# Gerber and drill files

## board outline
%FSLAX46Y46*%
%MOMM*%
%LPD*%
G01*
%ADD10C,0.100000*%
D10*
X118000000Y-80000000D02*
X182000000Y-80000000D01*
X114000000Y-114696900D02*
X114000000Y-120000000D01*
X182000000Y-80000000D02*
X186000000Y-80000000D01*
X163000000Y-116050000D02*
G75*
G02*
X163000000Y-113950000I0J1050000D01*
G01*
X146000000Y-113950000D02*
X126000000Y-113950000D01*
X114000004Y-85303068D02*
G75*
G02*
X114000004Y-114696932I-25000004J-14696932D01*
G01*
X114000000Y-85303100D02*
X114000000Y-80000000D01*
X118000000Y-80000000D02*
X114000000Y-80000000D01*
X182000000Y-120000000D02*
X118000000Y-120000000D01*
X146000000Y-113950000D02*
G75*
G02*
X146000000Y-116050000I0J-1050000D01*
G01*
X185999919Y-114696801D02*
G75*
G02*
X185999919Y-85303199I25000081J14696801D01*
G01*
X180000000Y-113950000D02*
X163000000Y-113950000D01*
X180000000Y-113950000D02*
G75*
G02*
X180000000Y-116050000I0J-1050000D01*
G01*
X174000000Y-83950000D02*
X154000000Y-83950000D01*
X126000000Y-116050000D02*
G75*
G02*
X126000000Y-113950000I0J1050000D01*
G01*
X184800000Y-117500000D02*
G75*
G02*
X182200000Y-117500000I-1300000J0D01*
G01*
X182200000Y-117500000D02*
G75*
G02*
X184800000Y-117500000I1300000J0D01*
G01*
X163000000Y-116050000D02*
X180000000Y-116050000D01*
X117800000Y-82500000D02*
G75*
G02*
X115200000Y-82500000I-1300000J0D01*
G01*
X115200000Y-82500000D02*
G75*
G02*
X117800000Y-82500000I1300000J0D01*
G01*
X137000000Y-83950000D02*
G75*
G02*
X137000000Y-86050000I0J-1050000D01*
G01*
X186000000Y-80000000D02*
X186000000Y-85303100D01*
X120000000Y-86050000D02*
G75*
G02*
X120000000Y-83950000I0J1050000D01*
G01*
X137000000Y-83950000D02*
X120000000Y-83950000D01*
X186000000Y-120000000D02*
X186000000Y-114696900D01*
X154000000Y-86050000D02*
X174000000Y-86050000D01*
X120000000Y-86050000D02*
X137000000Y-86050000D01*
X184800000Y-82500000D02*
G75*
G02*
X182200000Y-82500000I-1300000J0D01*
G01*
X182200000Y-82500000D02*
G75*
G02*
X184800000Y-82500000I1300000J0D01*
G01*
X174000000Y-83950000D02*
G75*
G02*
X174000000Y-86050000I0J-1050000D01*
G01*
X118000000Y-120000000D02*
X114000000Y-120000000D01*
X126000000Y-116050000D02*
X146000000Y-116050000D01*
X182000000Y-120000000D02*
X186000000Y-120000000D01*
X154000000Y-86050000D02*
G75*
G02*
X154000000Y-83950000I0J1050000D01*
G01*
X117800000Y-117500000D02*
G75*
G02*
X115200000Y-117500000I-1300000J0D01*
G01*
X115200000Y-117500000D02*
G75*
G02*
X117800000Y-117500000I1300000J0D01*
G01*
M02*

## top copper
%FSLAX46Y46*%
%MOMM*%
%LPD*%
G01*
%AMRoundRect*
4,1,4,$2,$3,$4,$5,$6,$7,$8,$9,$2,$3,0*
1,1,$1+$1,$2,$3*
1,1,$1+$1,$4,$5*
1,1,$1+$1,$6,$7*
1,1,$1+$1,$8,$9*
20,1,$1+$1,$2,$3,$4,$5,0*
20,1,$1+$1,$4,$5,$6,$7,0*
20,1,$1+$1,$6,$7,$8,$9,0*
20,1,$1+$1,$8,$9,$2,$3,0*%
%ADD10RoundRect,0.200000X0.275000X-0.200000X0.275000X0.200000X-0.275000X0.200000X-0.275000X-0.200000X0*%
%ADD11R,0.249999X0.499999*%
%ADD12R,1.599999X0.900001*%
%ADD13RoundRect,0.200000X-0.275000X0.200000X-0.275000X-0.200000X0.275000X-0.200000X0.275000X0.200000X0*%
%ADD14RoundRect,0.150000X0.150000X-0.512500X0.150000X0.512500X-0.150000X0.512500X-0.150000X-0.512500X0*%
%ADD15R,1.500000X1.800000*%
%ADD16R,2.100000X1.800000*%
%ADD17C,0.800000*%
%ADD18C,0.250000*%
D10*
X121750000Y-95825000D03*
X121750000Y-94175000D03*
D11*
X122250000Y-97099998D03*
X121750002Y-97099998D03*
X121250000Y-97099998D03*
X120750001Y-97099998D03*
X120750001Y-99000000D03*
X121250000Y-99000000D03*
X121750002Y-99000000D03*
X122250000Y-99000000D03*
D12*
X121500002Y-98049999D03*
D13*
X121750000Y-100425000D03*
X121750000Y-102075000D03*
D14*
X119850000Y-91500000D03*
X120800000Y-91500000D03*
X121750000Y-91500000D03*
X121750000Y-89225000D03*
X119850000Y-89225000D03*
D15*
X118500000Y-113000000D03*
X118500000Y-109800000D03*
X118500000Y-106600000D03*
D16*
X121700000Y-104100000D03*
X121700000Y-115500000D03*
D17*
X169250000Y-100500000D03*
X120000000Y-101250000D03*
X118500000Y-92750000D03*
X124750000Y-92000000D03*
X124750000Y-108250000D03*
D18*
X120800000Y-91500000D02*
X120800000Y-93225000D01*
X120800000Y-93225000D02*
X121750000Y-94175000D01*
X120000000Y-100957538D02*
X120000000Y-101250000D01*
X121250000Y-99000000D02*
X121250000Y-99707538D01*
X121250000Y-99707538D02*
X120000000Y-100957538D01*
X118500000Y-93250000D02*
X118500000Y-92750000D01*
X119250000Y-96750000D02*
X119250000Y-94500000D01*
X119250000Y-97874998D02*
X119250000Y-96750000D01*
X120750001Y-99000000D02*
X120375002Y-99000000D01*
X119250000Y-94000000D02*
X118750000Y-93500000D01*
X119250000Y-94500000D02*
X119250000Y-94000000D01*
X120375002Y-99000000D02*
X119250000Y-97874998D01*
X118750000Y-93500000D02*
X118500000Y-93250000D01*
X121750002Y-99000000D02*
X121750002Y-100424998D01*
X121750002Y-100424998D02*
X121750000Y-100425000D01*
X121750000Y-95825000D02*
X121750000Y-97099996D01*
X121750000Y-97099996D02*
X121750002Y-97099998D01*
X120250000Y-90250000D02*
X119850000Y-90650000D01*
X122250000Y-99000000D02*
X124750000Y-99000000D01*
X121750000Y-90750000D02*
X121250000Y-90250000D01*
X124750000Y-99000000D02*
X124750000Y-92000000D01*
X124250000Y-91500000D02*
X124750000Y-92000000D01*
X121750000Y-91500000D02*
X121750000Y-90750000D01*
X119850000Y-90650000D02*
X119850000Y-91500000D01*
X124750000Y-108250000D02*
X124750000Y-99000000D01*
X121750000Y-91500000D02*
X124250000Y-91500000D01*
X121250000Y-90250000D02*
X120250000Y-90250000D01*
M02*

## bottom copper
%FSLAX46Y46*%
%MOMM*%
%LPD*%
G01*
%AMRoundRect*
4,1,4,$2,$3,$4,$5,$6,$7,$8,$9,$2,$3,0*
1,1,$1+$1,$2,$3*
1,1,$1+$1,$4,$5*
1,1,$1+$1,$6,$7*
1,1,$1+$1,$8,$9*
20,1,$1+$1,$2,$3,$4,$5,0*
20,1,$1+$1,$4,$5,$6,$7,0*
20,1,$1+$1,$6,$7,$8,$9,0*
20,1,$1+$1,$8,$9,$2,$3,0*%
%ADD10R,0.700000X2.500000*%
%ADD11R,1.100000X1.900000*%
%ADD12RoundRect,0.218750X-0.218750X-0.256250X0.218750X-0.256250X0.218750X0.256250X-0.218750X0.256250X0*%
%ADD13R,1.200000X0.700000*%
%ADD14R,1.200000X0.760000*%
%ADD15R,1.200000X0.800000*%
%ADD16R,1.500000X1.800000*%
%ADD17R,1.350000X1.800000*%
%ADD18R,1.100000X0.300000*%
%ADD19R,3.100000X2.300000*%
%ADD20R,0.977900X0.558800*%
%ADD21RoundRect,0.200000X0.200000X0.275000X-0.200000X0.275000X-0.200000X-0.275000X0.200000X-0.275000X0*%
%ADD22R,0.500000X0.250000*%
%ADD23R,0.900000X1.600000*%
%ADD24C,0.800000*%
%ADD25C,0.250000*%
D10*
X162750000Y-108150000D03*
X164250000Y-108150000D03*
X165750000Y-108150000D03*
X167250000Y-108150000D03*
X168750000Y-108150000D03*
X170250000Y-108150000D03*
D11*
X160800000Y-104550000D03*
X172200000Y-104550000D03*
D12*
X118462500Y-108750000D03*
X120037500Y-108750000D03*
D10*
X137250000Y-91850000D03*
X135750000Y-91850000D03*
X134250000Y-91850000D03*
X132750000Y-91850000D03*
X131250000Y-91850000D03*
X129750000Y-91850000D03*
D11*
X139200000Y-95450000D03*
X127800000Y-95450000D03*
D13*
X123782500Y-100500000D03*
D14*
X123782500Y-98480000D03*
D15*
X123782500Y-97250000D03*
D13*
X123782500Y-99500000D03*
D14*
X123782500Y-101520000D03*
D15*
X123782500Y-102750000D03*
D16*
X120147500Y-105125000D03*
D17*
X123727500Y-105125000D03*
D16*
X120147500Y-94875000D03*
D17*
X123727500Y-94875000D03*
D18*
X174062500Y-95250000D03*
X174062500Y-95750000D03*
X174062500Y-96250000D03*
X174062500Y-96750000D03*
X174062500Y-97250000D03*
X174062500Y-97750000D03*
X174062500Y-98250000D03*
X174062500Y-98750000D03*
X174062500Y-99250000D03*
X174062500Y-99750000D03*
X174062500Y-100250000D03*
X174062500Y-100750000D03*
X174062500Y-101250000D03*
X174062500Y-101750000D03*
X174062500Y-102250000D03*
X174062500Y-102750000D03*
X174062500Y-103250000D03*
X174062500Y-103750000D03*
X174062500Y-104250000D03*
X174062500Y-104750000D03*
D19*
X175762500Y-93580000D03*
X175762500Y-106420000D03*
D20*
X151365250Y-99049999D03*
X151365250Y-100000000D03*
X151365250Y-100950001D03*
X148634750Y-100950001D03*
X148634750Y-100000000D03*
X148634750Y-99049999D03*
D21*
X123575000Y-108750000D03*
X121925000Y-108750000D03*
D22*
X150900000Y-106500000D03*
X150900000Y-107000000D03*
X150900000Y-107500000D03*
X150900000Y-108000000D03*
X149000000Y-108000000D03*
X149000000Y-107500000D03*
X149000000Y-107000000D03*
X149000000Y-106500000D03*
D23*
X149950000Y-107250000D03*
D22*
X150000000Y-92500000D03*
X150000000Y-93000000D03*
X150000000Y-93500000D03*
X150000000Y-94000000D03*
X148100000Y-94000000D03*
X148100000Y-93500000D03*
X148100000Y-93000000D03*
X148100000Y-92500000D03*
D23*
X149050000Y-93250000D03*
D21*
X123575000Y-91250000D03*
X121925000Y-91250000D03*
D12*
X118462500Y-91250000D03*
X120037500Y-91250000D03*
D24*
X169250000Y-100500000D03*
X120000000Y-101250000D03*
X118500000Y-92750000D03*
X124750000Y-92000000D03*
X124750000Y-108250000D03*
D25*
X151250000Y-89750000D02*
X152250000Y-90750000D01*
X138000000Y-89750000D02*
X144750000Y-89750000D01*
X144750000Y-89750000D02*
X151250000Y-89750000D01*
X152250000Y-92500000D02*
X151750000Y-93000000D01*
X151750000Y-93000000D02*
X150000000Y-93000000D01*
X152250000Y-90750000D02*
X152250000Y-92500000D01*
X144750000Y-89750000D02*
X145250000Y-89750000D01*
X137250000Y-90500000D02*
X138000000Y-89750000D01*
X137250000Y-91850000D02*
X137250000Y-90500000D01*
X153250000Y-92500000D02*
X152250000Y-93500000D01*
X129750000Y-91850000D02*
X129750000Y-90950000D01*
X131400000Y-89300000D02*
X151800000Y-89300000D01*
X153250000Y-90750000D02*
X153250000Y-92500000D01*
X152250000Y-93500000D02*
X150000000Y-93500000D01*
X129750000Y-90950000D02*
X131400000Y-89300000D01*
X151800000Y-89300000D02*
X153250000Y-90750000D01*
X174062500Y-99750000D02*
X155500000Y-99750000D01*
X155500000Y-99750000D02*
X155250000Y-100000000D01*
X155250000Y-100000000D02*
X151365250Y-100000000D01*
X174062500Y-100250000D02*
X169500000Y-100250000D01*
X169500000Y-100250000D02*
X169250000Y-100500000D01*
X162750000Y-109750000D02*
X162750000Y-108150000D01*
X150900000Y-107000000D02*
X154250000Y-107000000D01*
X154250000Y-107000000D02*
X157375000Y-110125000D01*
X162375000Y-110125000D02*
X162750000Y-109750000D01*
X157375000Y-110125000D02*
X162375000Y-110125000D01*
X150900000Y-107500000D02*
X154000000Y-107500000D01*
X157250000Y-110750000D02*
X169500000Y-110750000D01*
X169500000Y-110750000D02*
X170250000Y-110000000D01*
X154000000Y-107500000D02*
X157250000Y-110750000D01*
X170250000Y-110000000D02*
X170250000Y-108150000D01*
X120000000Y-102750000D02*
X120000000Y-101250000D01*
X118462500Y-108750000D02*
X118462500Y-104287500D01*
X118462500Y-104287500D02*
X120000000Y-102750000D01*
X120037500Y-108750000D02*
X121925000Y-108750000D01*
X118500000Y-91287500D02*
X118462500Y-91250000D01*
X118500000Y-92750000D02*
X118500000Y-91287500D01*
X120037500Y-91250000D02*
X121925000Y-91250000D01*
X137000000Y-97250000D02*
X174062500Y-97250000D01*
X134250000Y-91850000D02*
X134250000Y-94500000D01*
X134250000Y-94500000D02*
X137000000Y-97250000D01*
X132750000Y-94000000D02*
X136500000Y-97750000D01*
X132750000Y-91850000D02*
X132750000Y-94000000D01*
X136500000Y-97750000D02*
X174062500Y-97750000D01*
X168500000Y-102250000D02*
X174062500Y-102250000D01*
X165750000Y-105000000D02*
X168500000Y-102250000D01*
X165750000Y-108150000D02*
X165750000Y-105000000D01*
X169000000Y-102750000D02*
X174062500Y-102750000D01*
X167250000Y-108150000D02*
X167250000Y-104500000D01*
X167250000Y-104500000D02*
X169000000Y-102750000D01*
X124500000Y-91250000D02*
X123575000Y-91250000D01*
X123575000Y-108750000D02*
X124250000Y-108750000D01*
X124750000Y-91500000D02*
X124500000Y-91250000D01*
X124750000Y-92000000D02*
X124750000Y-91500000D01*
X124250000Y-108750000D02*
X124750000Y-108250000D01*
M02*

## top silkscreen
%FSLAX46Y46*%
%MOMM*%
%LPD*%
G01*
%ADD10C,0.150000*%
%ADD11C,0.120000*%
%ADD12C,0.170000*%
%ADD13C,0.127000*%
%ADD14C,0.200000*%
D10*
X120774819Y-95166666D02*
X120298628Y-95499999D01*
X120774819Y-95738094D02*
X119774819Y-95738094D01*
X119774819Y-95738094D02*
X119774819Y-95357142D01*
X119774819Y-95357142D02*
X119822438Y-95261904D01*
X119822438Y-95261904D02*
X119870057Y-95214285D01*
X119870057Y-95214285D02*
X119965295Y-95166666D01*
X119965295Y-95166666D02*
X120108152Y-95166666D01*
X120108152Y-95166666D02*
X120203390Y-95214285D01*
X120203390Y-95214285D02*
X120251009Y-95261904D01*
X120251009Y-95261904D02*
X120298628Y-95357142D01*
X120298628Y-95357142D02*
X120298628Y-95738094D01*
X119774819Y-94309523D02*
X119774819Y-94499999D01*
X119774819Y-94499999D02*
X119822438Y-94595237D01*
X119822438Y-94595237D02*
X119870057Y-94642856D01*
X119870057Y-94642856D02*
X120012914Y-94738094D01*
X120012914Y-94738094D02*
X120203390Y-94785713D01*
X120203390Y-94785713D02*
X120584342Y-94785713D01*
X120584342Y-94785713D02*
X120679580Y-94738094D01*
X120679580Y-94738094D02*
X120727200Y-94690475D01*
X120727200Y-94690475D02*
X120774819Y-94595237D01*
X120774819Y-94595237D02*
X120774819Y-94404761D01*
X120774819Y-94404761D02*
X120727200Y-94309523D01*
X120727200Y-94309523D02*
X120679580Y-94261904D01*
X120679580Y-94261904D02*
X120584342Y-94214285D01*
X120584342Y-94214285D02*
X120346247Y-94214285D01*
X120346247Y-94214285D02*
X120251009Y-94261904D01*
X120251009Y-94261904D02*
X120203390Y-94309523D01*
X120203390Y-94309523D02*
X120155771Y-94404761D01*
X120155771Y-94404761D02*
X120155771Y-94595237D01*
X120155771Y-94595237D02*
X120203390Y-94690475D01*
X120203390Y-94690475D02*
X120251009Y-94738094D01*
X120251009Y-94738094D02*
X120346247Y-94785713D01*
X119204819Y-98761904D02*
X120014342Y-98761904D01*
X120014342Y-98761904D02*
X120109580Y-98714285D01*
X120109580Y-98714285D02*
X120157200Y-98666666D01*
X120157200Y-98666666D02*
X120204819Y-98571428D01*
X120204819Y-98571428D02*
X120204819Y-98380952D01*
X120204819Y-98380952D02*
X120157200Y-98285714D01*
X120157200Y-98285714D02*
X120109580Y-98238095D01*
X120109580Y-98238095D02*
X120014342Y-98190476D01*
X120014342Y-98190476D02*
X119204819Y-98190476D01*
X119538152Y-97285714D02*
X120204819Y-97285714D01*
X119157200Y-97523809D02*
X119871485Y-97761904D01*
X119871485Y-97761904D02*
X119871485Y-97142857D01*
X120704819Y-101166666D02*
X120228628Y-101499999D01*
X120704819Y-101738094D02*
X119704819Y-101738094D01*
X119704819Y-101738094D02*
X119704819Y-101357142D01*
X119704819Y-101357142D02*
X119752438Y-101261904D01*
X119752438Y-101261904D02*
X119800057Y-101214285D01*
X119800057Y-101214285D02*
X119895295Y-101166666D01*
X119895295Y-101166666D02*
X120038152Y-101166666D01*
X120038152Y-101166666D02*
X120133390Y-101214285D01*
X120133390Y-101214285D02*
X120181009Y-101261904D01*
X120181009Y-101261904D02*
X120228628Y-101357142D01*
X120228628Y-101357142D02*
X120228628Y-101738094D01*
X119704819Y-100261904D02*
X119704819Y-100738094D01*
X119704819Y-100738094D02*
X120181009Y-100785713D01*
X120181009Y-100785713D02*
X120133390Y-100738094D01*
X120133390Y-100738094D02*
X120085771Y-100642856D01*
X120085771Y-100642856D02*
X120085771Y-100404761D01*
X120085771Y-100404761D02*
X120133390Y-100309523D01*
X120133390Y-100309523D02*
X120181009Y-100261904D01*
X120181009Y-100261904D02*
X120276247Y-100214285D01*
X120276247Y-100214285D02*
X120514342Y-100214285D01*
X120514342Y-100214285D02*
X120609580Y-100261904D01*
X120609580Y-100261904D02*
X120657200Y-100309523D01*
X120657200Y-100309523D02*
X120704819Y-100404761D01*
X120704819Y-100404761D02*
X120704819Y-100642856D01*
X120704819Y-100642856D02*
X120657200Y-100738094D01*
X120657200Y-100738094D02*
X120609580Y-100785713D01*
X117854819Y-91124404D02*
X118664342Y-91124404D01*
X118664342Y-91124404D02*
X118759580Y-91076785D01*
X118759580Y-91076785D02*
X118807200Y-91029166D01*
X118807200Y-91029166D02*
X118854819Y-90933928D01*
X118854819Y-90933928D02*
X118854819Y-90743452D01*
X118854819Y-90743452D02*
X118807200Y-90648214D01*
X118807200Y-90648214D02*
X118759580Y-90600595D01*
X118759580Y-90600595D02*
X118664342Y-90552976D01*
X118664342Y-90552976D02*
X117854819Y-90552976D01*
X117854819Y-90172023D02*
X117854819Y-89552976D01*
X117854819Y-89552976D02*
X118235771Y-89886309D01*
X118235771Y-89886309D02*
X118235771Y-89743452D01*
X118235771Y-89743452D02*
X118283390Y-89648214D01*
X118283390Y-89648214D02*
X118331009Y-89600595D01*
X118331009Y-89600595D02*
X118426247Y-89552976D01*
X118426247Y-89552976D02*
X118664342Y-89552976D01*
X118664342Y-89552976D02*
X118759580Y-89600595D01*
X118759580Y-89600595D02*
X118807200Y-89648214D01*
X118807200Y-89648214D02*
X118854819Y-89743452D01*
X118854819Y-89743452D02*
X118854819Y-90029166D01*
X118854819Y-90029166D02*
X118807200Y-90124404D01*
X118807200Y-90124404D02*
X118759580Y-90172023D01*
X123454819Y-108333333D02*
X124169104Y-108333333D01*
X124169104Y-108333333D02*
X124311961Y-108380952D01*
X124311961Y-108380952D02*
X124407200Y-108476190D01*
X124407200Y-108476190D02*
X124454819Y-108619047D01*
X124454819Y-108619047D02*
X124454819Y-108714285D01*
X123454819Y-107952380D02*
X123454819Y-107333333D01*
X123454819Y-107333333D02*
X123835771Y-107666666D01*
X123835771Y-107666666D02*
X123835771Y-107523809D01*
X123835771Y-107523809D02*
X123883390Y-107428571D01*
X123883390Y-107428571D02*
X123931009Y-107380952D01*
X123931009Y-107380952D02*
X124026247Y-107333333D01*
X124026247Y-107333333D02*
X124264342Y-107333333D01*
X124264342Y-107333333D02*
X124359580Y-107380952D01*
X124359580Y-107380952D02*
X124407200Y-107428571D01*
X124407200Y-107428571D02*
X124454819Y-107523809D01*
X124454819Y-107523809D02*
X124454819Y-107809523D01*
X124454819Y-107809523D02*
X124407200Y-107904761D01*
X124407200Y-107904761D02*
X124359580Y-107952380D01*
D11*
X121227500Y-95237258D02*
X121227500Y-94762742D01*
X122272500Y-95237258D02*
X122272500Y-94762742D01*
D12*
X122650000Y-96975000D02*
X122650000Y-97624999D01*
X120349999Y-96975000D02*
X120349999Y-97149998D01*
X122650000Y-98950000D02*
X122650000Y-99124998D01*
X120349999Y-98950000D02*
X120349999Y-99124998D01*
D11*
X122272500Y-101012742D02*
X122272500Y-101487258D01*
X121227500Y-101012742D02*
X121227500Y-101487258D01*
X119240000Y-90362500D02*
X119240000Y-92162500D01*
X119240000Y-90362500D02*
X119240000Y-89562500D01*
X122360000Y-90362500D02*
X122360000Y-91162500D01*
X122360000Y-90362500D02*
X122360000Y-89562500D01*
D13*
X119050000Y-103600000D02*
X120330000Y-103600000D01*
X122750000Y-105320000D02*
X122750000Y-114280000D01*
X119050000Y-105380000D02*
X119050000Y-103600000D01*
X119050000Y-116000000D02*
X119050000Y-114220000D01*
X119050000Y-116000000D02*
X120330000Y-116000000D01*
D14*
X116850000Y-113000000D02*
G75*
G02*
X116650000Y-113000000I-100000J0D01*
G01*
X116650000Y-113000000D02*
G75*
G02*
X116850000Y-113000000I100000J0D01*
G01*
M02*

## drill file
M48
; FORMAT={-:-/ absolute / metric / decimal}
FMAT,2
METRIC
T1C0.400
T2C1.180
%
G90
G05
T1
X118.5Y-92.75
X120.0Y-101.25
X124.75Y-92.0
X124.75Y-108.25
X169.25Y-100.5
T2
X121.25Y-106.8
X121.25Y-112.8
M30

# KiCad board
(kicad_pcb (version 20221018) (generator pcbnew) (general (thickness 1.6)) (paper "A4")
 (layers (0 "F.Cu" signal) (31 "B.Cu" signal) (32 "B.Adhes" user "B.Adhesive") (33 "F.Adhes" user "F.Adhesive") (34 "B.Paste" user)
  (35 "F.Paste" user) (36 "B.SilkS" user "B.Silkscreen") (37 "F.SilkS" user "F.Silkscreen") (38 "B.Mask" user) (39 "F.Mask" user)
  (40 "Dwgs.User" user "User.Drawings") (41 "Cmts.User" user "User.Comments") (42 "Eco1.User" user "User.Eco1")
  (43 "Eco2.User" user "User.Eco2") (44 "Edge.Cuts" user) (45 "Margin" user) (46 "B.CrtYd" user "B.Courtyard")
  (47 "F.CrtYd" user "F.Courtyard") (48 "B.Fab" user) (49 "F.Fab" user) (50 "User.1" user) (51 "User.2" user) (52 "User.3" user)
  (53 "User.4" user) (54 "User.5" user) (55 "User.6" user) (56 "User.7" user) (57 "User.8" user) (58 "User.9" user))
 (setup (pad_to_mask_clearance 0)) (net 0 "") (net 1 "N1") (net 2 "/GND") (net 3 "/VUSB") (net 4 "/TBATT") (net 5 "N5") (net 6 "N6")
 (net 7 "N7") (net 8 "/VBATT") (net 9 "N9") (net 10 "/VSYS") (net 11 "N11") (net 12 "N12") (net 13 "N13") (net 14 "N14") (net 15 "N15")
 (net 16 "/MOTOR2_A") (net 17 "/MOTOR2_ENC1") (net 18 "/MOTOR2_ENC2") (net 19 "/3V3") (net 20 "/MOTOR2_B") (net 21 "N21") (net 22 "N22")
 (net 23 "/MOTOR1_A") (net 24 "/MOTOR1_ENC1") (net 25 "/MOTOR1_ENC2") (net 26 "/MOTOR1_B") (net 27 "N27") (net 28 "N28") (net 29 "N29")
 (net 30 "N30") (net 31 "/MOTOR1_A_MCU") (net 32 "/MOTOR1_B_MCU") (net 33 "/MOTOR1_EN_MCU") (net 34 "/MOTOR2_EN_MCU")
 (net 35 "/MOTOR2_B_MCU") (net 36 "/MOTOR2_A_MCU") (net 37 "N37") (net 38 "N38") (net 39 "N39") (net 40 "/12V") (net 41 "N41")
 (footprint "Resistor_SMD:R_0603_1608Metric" (layer "F.Cu") (at 121.75 95 90)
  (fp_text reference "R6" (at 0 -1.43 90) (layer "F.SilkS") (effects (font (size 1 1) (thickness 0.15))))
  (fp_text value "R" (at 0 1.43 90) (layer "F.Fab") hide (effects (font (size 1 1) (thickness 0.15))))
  (fp_line (start -0.237258 -0.5225) (end 0.237258 -0.5225) (stroke (width 0.12) (type solid)) (layer "F.SilkS"))
  (fp_line (start -0.237258 0.5225) (end 0.237258 0.5225) (stroke (width 0.12) (type solid)) (layer "F.SilkS"))
  (pad "1" smd roundrect (at -0.825 0 90) (size 0.8 0.95) (layers "F.Cu" "F.Paste" "F.Mask") (roundrect_rratio 0.25) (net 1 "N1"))
  (pad "2" smd roundrect (at 0.825 0 90) (size 0.8 0.95) (layers "F.Cu" "F.Paste" "F.Mask") (roundrect_rratio 0.25) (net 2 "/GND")))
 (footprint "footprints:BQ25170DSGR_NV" (layer "F.Cu") (at 121.500002 98.049999 -90)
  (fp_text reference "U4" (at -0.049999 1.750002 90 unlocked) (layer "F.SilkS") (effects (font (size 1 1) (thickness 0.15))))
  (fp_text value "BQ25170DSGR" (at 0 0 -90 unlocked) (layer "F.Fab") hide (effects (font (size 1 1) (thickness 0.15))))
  (fp_line (start -1.074999 -1.149998) (end -0.425 -1.149998) (stroke (width 0.17) (type solid)) (layer "F.SilkS"))
  (fp_line (start -1.074999 1.150003) (end -0.900001 1.150003) (stroke (width 0.17) (type solid)) (layer "F.SilkS"))
  (fp_line (start 0.900001 -1.149998) (end 1.074999 -1.149998) (stroke (width 0.17) (type solid)) (layer "F.SilkS"))
  (fp_line (start 0.900001 1.150003) (end 1.074999 1.150003) (stroke (width 0.17) (type solid)) (layer "F.SilkS"))
  (pad "1" smd rect (at -0.950001 -0.749998) (size 0.249999 0.499999) (layers "F.Cu" "F.Paste" "F.Mask") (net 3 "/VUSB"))
  (pad "2" smd rect (at -0.950001 -0.25) (size 0.249999 0.499999) (layers "F.Cu" "F.Paste" "F.Mask") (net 1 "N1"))
  (pad "3" smd rect (at -0.950001 0.250002) (size 0.249999 0.499999) (layers "F.Cu" "F.Paste" "F.Mask") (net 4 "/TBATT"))
  (pad "4" smd rect (at -0.950001 0.750001) (size 0.249999 0.499999) (layers "F.Cu" "F.Paste" "F.Mask") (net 2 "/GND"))
  (pad "5" smd rect (at 0.950001 0.750001) (size 0.249999 0.499999) (layers "F.Cu" "F.Paste" "F.Mask") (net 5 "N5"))
  (pad "6" smd rect (at 0.950001 0.250002) (size 0.249999 0.499999) (layers "F.Cu" "F.Paste" "F.Mask") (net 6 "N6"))
  (pad "7" smd rect (at 0.950001 -0.25) (size 0.249999 0.499999) (layers "F.Cu" "F.Paste" "F.Mask") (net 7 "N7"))
  (pad "8" smd rect (at 0.950001 -0.749998) (size 0.249999 0.499999) (layers "F.Cu" "F.Paste" "F.Mask") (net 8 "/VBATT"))
  (pad "9" smd rect (at 0 0 270) (size 0.900001 1.599999) (layers "F.Cu" "F.Paste" "F.Mask") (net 2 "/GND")))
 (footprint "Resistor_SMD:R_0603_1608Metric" (layer "F.Cu") (at 121.75 101.25 -90)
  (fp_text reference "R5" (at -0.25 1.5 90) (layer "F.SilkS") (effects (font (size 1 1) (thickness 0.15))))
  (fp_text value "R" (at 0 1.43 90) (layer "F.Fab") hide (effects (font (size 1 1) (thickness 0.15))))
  (fp_line (start -0.237258 -0.5225) (end 0.237258 -0.5225) (stroke (width 0.12) (type solid)) (layer "F.SilkS"))
  (fp_line (start -0.237258 0.5225) (end 0.237258 0.5225) (stroke (width 0.12) (type solid)) (layer "F.SilkS"))
  (pad "1" smd roundrect (at -0.825 0 270) (size 0.8 0.95) (layers "F.Cu" "F.Paste" "F.Mask") (roundrect_rratio 0.25) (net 7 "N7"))
  (pad "2" smd roundrect (at 0.825 0 270) (size 0.8 0.95) (layers "F.Cu" "F.Paste" "F.Mask") (roundrect_rratio 0.25) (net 2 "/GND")))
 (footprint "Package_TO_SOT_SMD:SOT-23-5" (layer "F.Cu") (at 120.8 90.3625 90)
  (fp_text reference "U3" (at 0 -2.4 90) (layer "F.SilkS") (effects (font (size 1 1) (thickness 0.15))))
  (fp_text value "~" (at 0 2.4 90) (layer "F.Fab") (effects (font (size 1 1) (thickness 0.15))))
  (fp_line (start 0 -1.56) (end -1.8 -1.56) (stroke (width 0.12) (type solid)) (layer "F.SilkS"))
  (fp_line (start 0 -1.56) (end 0.8 -1.56) (stroke (width 0.12) (type solid)) (layer "F.SilkS"))
  (fp_line (start 0 1.56) (end -0.8 1.56) (stroke (width 0.12) (type solid)) (layer "F.SilkS"))
  (fp_line (start 0 1.56) (end 0.8 1.56) (stroke (width 0.12) (type solid)) (layer "F.SilkS"))
  (pad "1" smd roundrect (at -1.1375 -0.95 90) (size 1.325 0.6) (layers "F.Cu" "F.Paste" "F.Mask") (roundrect_rratio 0.25) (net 8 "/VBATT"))
  (pad "2" smd roundrect (at -1.1375 0 90) (size 1.325 0.6) (layers "F.Cu" "F.Paste" "F.Mask") (roundrect_rratio 0.25) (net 2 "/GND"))
  (pad "3" smd roundrect (at -1.1375 0.95 90) (size 1.325 0.6) (layers "F.Cu" "F.Paste" "F.Mask") (roundrect_rratio 0.25) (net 8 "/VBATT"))
  (pad "4" smd roundrect (at 1.1375 0.95 90) (size 1.325 0.6) (layers "F.Cu" "F.Paste" "F.Mask") (roundrect_rratio 0.25) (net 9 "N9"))
  (pad "5" smd roundrect (at 1.1375 -0.95 90) (size 1.325 0.6) (layers "F.Cu" "F.Paste" "F.Mask") (roundrect_rratio 0.25) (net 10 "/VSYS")))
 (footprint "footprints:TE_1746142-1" (layer "F.Cu") (at 121.25 109.8 -90)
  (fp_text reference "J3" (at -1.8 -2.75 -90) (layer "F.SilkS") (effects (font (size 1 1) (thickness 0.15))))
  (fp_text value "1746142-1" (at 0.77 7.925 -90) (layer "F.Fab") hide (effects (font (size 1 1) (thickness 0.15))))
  (fp_line (start -6.2 2.2) (end -6.2 0.92) (stroke (width 0.127) (type solid)) (layer "F.SilkS"))
  (fp_line (start -4.48 -1.5) (end 4.48 -1.5) (stroke (width 0.127) (type solid)) (layer "F.SilkS"))
  (fp_line (start -4.42 2.2) (end -6.2 2.2) (stroke (width 0.127) (type solid)) (layer "F.SilkS"))
  (fp_line (start 6.2 2.2) (end 4.42 2.2) (stroke (width 0.127) (type solid)) (layer "F.SilkS"))
  (fp_line (start 6.2 2.2) (end 6.2 0.92) (stroke (width 0.127) (type solid)) (layer "F.SilkS"))
  (fp_circle (center 3.2 4.5) (end 3.3 4.5) (stroke (width 0.2) (type solid)) (fill none) (layer "F.SilkS"))
  (pad "" np_thru_hole circle (at -3 0 270) (size 1.18 1.18) (drill 1.18) (layers "*.Cu" "*.Mask"))
  (pad "" np_thru_hole circle (at 3 0 270) (size 1.18 1.18) (drill 1.18) (layers "*.Cu" "*.Mask"))
  (pad "1" smd rect (at 3.2 2.75 270) (size 1.8 1.5) (layers "F.Cu" "F.Paste" "F.Mask") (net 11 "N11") (solder_mask_margin 0.102))
  (pad "2" smd rect (at 0 2.75 270) (size 1.8 1.5) (layers "F.Cu" "F.Paste" "F.Mask") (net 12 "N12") (solder_mask_margin 0.102))
  (pad "3" smd rect (at -3.2 2.75 270) (size 1.8 1.5) (layers "F.Cu" "F.Paste" "F.Mask") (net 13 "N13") (solder_mask_margin 0.102))
  (pad "SH1" smd rect (at -5.7 -0.45 270) (size 1.8 2.1) (layers "F.Cu" "F.Paste" "F.Mask") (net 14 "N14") (solder_mask_margin 0.102))
  (pad "SH2" smd rect (at 5.7 -0.45 270) (size 1.8 2.1) (layers "F.Cu" "F.Paste" "F.Mask") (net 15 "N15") (solder_mask_margin 0.102)))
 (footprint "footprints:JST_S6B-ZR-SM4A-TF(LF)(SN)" (layer "B.Cu") (at 166.5 108.15)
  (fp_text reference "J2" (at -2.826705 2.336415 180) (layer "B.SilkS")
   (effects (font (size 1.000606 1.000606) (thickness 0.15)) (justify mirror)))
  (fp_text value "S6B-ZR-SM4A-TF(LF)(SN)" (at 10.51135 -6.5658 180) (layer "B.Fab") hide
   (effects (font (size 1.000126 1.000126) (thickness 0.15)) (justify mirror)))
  (pad "1" smd rect (at -3.75 0) (size 0.7 2.5) (layers "B.Cu" "B.Paste" "B.Mask") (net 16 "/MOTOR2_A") (solder_mask_margin 0.102))
  (pad "2" smd rect (at -2.25 0) (size 0.7 2.5) (layers "B.Cu" "B.Paste" "B.Mask") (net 2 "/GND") (solder_mask_margin 0.102))
  (pad "3" smd rect (at -0.75 0) (size 0.7 2.5) (layers "B.Cu" "B.Paste" "B.Mask") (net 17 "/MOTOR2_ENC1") (solder_mask_margin 0.102))
  (pad "4" smd rect (at 0.75 0) (size 0.7 2.5) (layers "B.Cu" "B.Paste" "B.Mask") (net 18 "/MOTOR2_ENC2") (solder_mask_margin 0.102))
  (pad "5" smd rect (at 2.25 0) (size 0.7 2.5) (layers "B.Cu" "B.Paste" "B.Mask") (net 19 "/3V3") (solder_mask_margin 0.102))
  (pad "6" smd rect (at 3.75 0) (size 0.7 2.5) (layers "B.Cu" "B.Paste" "B.Mask") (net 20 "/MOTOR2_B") (solder_mask_margin 0.102))
  (pad "SH1" smd rect (at -5.7 -3.6) (size 1.1 1.9) (layers "B.Cu" "B.Paste" "B.Mask") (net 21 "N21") (solder_mask_margin 0.102))
  (pad "SH2" smd rect (at 5.7 -3.6) (size 1.1 1.9) (layers "B.Cu" "B.Paste" "B.Mask") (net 21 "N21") (solder_mask_margin 0.102)))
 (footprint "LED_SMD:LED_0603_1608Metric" (layer "B.Cu") (at 119.25 108.75)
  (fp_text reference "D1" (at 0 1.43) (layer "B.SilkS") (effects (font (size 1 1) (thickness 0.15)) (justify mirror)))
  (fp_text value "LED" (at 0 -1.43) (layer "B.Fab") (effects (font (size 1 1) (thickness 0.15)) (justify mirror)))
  (pad "1" smd roundrect (at -0.7875 0) (size 0.875 0.95) (layers "B.Cu" "B.Paste" "B.Mask") (roundrect_rratio 0.25) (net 6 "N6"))
  (pad "2" smd roundrect (at 0.7875 0) (size 0.875 0.95) (layers "B.Cu" "B.Paste" "B.Mask") (roundrect_rratio 0.25) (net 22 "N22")))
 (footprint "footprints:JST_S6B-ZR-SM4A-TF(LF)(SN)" (layer "B.Cu") (at 133.5 91.85 180)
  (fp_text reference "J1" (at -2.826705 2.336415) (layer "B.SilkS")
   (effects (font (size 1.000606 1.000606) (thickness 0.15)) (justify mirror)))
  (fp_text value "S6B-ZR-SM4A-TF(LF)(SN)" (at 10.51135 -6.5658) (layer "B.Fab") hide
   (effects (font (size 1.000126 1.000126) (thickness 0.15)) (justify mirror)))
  (pad "1" smd rect (at -3.75 0 180) (size 0.7 2.5) (layers "B.Cu" "B.Paste" "B.Mask") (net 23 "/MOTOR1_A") (solder_mask_margin 0.102))
  (pad "2" smd rect (at -2.25 0 180) (size 0.7 2.5) (layers "B.Cu" "B.Paste" "B.Mask") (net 2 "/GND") (solder_mask_margin 0.102))
  (pad "3" smd rect (at -0.75 0 180) (size 0.7 2.5) (layers "B.Cu" "B.Paste" "B.Mask") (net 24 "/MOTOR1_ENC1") (solder_mask_margin 0.102))
  (pad "4" smd rect (at 0.75 0 180) (size 0.7 2.5) (layers "B.Cu" "B.Paste" "B.Mask") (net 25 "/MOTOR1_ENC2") (solder_mask_margin 0.102))
  (pad "5" smd rect (at 2.25 0 180) (size 0.7 2.5) (layers "B.Cu" "B.Paste" "B.Mask") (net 19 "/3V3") (solder_mask_margin 0.102))
  (pad "6" smd rect (at 3.75 0 180) (size 0.7 2.5) (layers "B.Cu" "B.Paste" "B.Mask") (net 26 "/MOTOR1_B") (solder_mask_margin 0.102))
  (pad "SH1" smd rect (at -5.7 -3.6 180) (size 1.1 1.9) (layers "B.Cu" "B.Paste" "B.Mask") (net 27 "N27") (solder_mask_margin 0.102))
  (pad "SH2" smd rect (at 5.7 -3.6 180) (size 1.1 1.9) (layers "B.Cu" "B.Paste" "B.Mask") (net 27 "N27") (solder_mask_margin 0.102)))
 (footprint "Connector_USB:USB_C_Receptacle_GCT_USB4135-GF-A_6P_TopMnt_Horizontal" (layer "B.Cu") (at 120.75 100 90)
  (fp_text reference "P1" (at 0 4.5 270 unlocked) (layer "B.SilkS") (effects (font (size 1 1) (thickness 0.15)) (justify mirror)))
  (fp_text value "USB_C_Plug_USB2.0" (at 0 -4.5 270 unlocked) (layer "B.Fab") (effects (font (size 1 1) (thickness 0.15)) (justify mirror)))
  (pad "A5" smd rect (at -0.5 3.0325 90) (size 0.7 1.2) (layers "B.Cu" "B.Paste" "B.Mask") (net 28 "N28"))
  (pad "A9" smd rect (at 1.52 3.0325 270) (size 0.76 1.2) (layers "B.Cu" "B.Paste" "B.Mask") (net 3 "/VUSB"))
  (pad "A12" smd rect (at 2.75 3.0325 270) (size 0.8 1.2) (layers "B.Cu" "B.Paste" "B.Mask") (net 2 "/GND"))
  (pad "B5" smd rect (at 0.5 3.0325 270) (size 0.7 1.2) (layers "B.Cu" "B.Paste" "B.Mask") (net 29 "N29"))
  (pad "B9" smd rect (at -1.52 3.0325 90) (size 0.76 1.2) (layers "B.Cu" "B.Paste" "B.Mask") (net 3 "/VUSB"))
  (pad "B12" smd rect (at -2.75 3.0325 90) (size 0.8 1.2) (layers "B.Cu" "B.Paste" "B.Mask") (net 2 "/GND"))
  (pad "S1" smd rect (at -5.125 -0.6025 90) (size 1.8 1.5) (layers "B.Cu" "B.Paste" "B.Mask") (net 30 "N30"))
  (pad "S1" smd rect (at -5.125 2.9775 90) (size 1.8 1.35) (layers "B.Cu" "B.Paste" "B.Mask") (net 30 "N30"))
  (pad "S1" smd rect (at 5.125 -0.6025 90) (size 1.8 1.5) (layers "B.Cu" "B.Paste" "B.Mask") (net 30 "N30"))
  (pad "S1" smd rect (at 5.125 2.9775 90) (size 1.8 1.35) (layers "B.Cu" "B.Paste" "B.Mask") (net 30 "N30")))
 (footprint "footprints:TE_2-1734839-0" (layer "B.Cu") (at 174.0625 100 -90)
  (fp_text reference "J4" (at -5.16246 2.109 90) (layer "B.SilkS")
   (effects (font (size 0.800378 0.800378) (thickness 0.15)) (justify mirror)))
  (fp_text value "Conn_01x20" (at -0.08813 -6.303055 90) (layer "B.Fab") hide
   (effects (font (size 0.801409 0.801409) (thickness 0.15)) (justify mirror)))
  (pad "1" smd rect (at -4.75 0 270) (size 0.3 1.1) (layers "B.Cu" "B.Paste" "B.Mask") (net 10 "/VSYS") (solder_mask_margin 0.102))
  (pad "2" smd rect (at -4.25 0 270) (size 0.3 1.1) (layers "B.Cu" "B.Paste" "B.Mask") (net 10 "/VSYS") (solder_mask_margin 0.102))
  (pad "3" smd rect (at -3.75 0 270) (size 0.3 1.1) (layers "B.Cu" "B.Paste" "B.Mask") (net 2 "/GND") (solder_mask_margin 0.102))
  (pad "4" smd rect (at -3.25 0 270) (size 0.3 1.1) (layers "B.Cu" "B.Paste" "B.Mask") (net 2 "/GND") (solder_mask_margin 0.102))
  (pad "5" smd rect (at -2.75 0 270) (size 0.3 1.1) (layers "B.Cu" "B.Paste" "B.Mask") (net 24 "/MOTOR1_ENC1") (solder_mask_margin 0.102))
  (pad "6" smd rect (at -2.25 0 270) (size 0.3 1.1) (layers "B.Cu" "B.Paste" "B.Mask") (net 25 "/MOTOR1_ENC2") (solder_mask_margin 0.102))
  (pad "7" smd rect (at -1.75 0 270) (size 0.3 1.1) (layers "B.Cu" "B.Paste" "B.Mask") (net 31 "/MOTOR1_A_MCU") (solder_mask_margin 0.102))
  (pad "8" smd rect (at -1.25 0 270) (size 0.3 1.1) (layers "B.Cu" "B.Paste" "B.Mask") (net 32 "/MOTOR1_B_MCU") (solder_mask_margin 0.102))
  (pad "9" smd rect (at -0.75 0 270) (size 0.3 1.1) (layers "B.Cu" "B.Paste" "B.Mask") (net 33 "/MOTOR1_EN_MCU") (solder_mask_margin 0.102))
  (pad "10" smd rect (at -0.25 0 270) (size 0.3 1.1) (layers "B.Cu" "B.Paste" "B.Mask") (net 2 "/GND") (solder_mask_margin 0.102))
  (pad "11" smd rect (at 0.25 0 270) (size 0.3 1.1) (layers "B.Cu" "B.Paste" "B.Mask") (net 19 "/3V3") (solder_mask_margin 0.102))
  (pad "12" smd rect (at 0.75 0 270) (size 0.3 1.1) (layers "B.Cu" "B.Paste" "B.Mask") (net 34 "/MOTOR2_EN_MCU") (solder_mask_margin 0.102))
  (pad "13" smd rect (at 1.25 0 270) (size 0.3 1.1) (layers "B.Cu" "B.Paste" "B.Mask") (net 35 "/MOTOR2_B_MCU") (solder_mask_margin 0.102))
  (pad "14" smd rect (at 1.75 0 270) (size 0.3 1.1) (layers "B.Cu" "B.Paste" "B.Mask") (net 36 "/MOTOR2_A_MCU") (solder_mask_margin 0.102))
  (pad "15" smd rect (at 2.25 0 270) (size 0.3 1.1) (layers "B.Cu" "B.Paste" "B.Mask") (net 17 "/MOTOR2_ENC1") (solder_mask_margin 0.102))
  (pad "16" smd rect (at 2.75 0 270) (size 0.3 1.1) (layers "B.Cu" "B.Paste" "B.Mask") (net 18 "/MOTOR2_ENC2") (solder_mask_margin 0.102))
  (pad "17" smd rect (at 3.25 0 270) (size 0.3 1.1) (layers "B.Cu" "B.Paste" "B.Mask") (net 2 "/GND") (solder_mask_margin 0.102))
  (pad "18" smd rect (at 3.75 0 270) (size 0.3 1.1) (layers "B.Cu" "B.Paste" "B.Mask") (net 2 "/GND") (solder_mask_margin 0.102))
  (pad "19" smd rect (at 4.25 0 270) (size 0.3 1.1) (layers "B.Cu" "B.Paste" "B.Mask") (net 3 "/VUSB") (solder_mask_margin 0.102))
  (pad "20" smd rect (at 4.75 0 270) (size 0.3 1.1) (layers "B.Cu" "B.Paste" "B.Mask") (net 3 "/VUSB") (solder_mask_margin 0.102))
  (pad "S1" smd rect (at -6.42 -1.7 270) (size 2.3 3.1) (layers "B.Cu" "B.Paste" "B.Mask") (solder_mask_margin 0.102))
  (pad "S2" smd rect (at 6.42 -1.7 270) (size 2.3 3.1) (layers "B.Cu" "B.Paste" "B.Mask") (solder_mask_margin 0.102)))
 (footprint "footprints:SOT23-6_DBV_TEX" (layer "B.Cu") (at 150 100 180)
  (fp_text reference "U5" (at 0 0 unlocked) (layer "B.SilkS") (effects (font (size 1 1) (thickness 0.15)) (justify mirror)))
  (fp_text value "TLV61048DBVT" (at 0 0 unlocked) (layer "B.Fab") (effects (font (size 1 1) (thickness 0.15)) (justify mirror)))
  (pad "1" smd rect (at -1.36525 0.950001 180) (size 0.9779 0.5588) (layers "B.Cu" "B.Paste" "B.Mask") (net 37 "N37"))
  (pad "2" smd rect (at -1.36525 0 180) (size 0.9779 0.5588) (layers "B.Cu" "B.Paste" "B.Mask") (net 2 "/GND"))
  (pad "3" smd rect (at -1.36525 -0.950001 180) (size 0.9779 0.5588) (layers "B.Cu" "B.Paste" "B.Mask") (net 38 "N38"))
  (pad "4" smd rect (at 1.36525 -0.950001 180) (size 0.9779 0.5588) (layers "B.Cu" "B.Paste" "B.Mask") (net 10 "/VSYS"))
  (pad "5" smd rect (at 1.36525 0 180) (size 0.9779 0.5588) (layers "B.Cu" "B.Paste" "B.Mask") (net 10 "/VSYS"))
  (pad "6" smd rect (at 1.36525 0.950001 180) (size 0.9779 0.5588) (layers "B.Cu" "B.Paste" "B.Mask") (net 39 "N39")))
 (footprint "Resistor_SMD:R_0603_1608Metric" (layer "B.Cu") (at 122.75 108.75 180)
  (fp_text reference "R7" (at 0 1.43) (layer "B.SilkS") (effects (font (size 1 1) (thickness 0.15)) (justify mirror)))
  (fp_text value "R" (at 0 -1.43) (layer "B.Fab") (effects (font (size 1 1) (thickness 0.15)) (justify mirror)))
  (pad "1" smd roundrect (at -0.825 0 180) (size 0.8 0.95) (layers "B.Cu" "B.Paste" "B.Mask") (roundrect_rratio 0.25) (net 8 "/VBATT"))
  (pad "2" smd roundrect (at 0.825 0 180) (size 0.8 0.95) (layers "B.Cu" "B.Paste" "B.Mask") (roundrect_rratio 0.25) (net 22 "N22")))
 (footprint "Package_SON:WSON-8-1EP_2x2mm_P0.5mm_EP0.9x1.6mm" (layer "B.Cu") (at 149.95 107.25 180)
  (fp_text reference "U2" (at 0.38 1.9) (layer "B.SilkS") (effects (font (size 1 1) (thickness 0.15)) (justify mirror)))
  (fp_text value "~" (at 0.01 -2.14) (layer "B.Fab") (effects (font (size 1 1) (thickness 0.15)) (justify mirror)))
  (pad "" smd rect (at 0 -0.4 180) (size 0.75 0.65) (layers "B.Paste"))
  (pad "" smd rect (at 0 0.4 180) (size 0.75 0.65) (layers "B.Paste"))
  (pad "1" smd rect (at -0.95 0.75 180) (size 0.5 0.25) (layers "B.Cu" "B.Paste" "B.Mask") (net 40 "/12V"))
  (pad "2" smd rect (at -0.95 0.25 180) (size 0.5 0.25) (layers "B.Cu" "B.Paste" "B.Mask") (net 16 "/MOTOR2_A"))
  (pad "3" smd rect (at -0.95 -0.25 180) (size 0.5 0.25) (layers "B.Cu" "B.Paste" "B.Mask") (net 20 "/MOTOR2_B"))
  (pad "4" smd rect (at -0.95 -0.75 180) (size 0.5 0.25) (layers "B.Cu" "B.Paste" "B.Mask") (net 2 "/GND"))
  (pad "5" smd rect (at 0.95 -0.75 180) (size 0.5 0.25) (layers "B.Cu" "B.Paste" "B.Mask") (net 35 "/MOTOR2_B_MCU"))
  (pad "6" smd rect (at 0.95 -0.25 180) (size 0.5 0.25) (layers "B.Cu" "B.Paste" "B.Mask") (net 36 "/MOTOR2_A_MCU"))
  (pad "7" smd rect (at 0.95 0.25 180) (size 0.5 0.25) (layers "B.Cu" "B.Paste" "B.Mask") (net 34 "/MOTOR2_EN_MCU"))
  (pad "8" smd rect (at 0.95 0.75 180) (size 0.5 0.25) (layers "B.Cu" "B.Paste" "B.Mask") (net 19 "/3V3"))
  (pad "9" smd rect (at 0 0 180) (size 0.9 1.6) (layers "B.Cu" "B.Mask") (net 2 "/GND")))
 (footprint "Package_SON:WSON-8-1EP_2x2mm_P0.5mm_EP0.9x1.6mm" (layer "B.Cu") (at 149.05 93.25 180)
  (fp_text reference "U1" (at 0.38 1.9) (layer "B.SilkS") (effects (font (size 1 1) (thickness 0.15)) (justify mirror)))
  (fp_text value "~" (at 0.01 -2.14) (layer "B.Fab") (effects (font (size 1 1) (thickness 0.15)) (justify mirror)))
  (pad "" smd rect (at 0 -0.4 180) (size 0.75 0.65) (layers "B.Paste"))
  (pad "" smd rect (at 0 0.4 180) (size 0.75 0.65) (layers "B.Paste"))
  (pad "1" smd rect (at -0.95 0.75 180) (size 0.5 0.25) (layers "B.Cu" "B.Paste" "B.Mask") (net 40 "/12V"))
  (pad "2" smd rect (at -0.95 0.25 180) (size 0.5 0.25) (layers "B.Cu" "B.Paste" "B.Mask") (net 23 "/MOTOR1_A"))
  (pad "3" smd rect (at -0.95 -0.25 180) (size 0.5 0.25) (layers "B.Cu" "B.Paste" "B.Mask") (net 26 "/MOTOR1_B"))
  (pad "4" smd rect (at -0.95 -0.75 180) (size 0.5 0.25) (layers "B.Cu" "B.Paste" "B.Mask") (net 2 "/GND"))
  (pad "5" smd rect (at 0.95 -0.75 180) (size 0.5 0.25) (layers "B.Cu" "B.Paste" "B.Mask") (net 32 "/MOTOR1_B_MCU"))
  (pad "6" smd rect (at 0.95 -0.25 180) (size 0.5 0.25) (layers "B.Cu" "B.Paste" "B.Mask") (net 31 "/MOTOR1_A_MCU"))
  (pad "7" smd rect (at 0.95 0.25 180) (size 0.5 0.25) (layers "B.Cu" "B.Paste" "B.Mask") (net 33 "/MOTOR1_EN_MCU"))
  (pad "8" smd rect (at 0.95 0.75 180) (size 0.5 0.25) (layers "B.Cu" "B.Paste" "B.Mask") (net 19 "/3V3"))
  (pad "9" smd rect (at 0 0 180) (size 0.9 1.6) (layers "B.Cu" "B.Mask") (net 2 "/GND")))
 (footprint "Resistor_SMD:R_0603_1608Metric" (layer "B.Cu") (at 122.75 91.25 180)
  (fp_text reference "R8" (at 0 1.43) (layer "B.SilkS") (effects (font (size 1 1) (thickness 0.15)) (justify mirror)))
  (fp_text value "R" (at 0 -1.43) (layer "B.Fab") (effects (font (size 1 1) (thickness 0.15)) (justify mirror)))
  (pad "1" smd roundrect (at -0.825 0 180) (size 0.8 0.95) (layers "B.Cu" "B.Paste" "B.Mask") (roundrect_rratio 0.25) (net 8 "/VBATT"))
  (pad "2" smd roundrect (at 0.825 0 180) (size 0.8 0.95) (layers "B.Cu" "B.Paste" "B.Mask") (roundrect_rratio 0.25) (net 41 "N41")))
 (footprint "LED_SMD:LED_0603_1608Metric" (layer "B.Cu") (at 119.25 91.25)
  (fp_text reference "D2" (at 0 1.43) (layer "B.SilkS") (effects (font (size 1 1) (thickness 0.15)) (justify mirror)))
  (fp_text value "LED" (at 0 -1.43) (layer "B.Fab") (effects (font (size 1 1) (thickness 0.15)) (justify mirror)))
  (pad "1" smd roundrect (at -0.7875 0) (size 0.875 0.95) (layers "B.Cu" "B.Paste" "B.Mask") (roundrect_rratio 0.25) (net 5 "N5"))
  (pad "2" smd roundrect (at 0.7875 0) (size 0.875 0.95) (layers "B.Cu" "B.Paste" "B.Mask") (roundrect_rratio 0.25) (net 41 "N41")))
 (gr_line (start 118 80) (end 182 80) (stroke (width 0.1) (type solid)) (layer "Edge.Cuts"))
 (gr_line (start 114 114.6969) (end 114 120) (stroke (width 0.1) (type solid)) (layer "Edge.Cuts"))
 (gr_line (start 182 80) (end 186 80) (stroke (width 0.1) (type solid)) (layer "Edge.Cuts"))
 (gr_arc (start 163 116.05) (mid 161.95 115) (end 163 113.95) (stroke (width 0.1) (type solid)) (layer "Edge.Cuts"))
 (gr_line (start 146 113.95) (end 126 113.95) (stroke (width 0.1) (type solid)) (layer "Edge.Cuts"))
 (gr_arc (start 114.000004 85.303068) (mid 118 100) (end 114.000004 114.696932) (stroke (width 0.1) (type solid)) (layer "Edge.Cuts"))
 (gr_line (start 114 85.3031) (end 114 80) (stroke (width 0.1) (type solid)) (layer "Edge.Cuts"))
 (gr_line (start 118 80) (end 114 80) (stroke (width 0.1) (type solid)) (layer "Edge.Cuts"))
 (gr_line (start 182 120) (end 118 120) (stroke (width 0.1) (type solid)) (layer "Edge.Cuts"))
 (gr_arc (start 146 113.95) (mid 147.05 115) (end 146 116.05) (stroke (width 0.1) (type solid)) (layer "Edge.Cuts"))
 (gr_arc (start 185.999919 114.696801) (mid 182 100) (end 185.999919 85.303199) (stroke (width 0.1) (type solid)) (layer "Edge.Cuts"))
 (gr_line (start 180 113.95) (end 163 113.95) (stroke (width 0.1) (type solid)) (layer "Edge.Cuts"))
 (gr_arc (start 180 113.95) (mid 181.05 115) (end 180 116.05) (stroke (width 0.1) (type solid)) (layer "Edge.Cuts"))
 (gr_line (start 174 83.95) (end 154 83.95) (stroke (width 0.1) (type solid)) (layer "Edge.Cuts"))
 (gr_arc (start 126 116.05) (mid 124.95 115) (end 126 113.95) (stroke (width 0.1) (type solid)) (layer "Edge.Cuts"))
 (gr_circle (center 183.5 117.5) (end 184.8 117.5) (stroke (width 0.1) (type solid)) (fill none) (layer "Edge.Cuts"))
 (gr_line (start 163 116.05) (end 180 116.05) (stroke (width 0.1) (type solid)) (layer "Edge.Cuts"))
 (gr_circle (center 116.5 82.5) (end 117.8 82.5) (stroke (width 0.1) (type solid)) (fill none) (layer "Edge.Cuts"))
 (gr_arc (start 137 83.95) (mid 138.05 85) (end 137 86.05) (stroke (width 0.1) (type solid)) (layer "Edge.Cuts"))
 (gr_line (start 186 80) (end 186 85.3031) (stroke (width 0.1) (type solid)) (layer "Edge.Cuts"))
 (gr_arc (start 120 86.05) (mid 118.95 85) (end 120 83.95) (stroke (width 0.1) (type solid)) (layer "Edge.Cuts"))
 (gr_line (start 137 83.95) (end 120 83.95) (stroke (width 0.1) (type solid)) (layer "Edge.Cuts"))
 (gr_line (start 186 120) (end 186 114.6969) (stroke (width 0.1) (type solid)) (layer "Edge.Cuts"))
 (gr_line (start 154 86.05) (end 174 86.05) (stroke (width 0.1) (type solid)) (layer "Edge.Cuts"))
 (gr_line (start 120 86.05) (end 137 86.05) (stroke (width 0.1) (type solid)) (layer "Edge.Cuts"))
 (gr_circle (center 183.5 82.5) (end 184.8 82.5) (stroke (width 0.1) (type solid)) (fill none) (layer "Edge.Cuts"))
 (gr_arc (start 174 83.95) (mid 175.05 85) (end 174 86.05) (stroke (width 0.1) (type solid)) (layer "Edge.Cuts"))
 (gr_line (start 118 120) (end 114 120) (stroke (width 0.1) (type solid)) (layer "Edge.Cuts"))
 (gr_line (start 126 116.05) (end 146 116.05) (stroke (width 0.1) (type solid)) (layer "Edge.Cuts"))
 (gr_line (start 182 120) (end 186 120) (stroke (width 0.1) (type solid)) (layer "Edge.Cuts"))
 (gr_arc (start 154 86.05) (mid 152.95 85) (end 154 83.95) (stroke (width 0.1) (type solid)) (layer "Edge.Cuts"))
 (gr_circle (center 116.5 117.5) (end 117.8 117.5) (stroke (width 0.1) (type solid)) (fill none) (layer "Edge.Cuts"))
 (segment (start 151.25 89.75) (end 152.25 90.75) (width 0.25) (layer "B.Cu") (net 23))
 (segment (start 138 89.75) (end 144.75 89.75) (width 0.25) (layer "B.Cu") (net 23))
 (segment (start 144.75 89.75) (end 151.25 89.75) (width 0.25) (layer "B.Cu") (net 23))
 (segment (start 152.25 92.5) (end 151.75 93) (width 0.25) (layer "B.Cu") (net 23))
 (segment (start 151.75 93) (end 150 93) (width 0.25) (layer "B.Cu") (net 23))
 (segment (start 152.25 90.75) (end 152.25 92.5) (width 0.25) (layer "B.Cu") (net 23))
 (segment (start 144.75 89.75) (end 145.25 89.75) (width 0.25) (layer "B.Cu") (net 23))
 (segment (start 137.25 90.5) (end 138 89.75) (width 0.25) (layer "B.Cu") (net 23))
 (segment (start 137.25 91.85) (end 137.25 90.5) (width 0.25) (layer "B.Cu") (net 23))
 (segment (start 153.25 92.5) (end 152.25 93.5) (width 0.25) (layer "B.Cu") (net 26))
 (segment (start 129.75 91.85) (end 129.75 90.95) (width 0.25) (layer "B.Cu") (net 26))
 (segment (start 131.4 89.3) (end 151.8 89.3) (width 0.25) (layer "B.Cu") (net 26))
 (segment (start 153.25 90.75) (end 153.25 92.5) (width 0.25) (layer "B.Cu") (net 26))
 (segment (start 152.25 93.5) (end 150 93.5) (width 0.25) (layer "B.Cu") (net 26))
 (segment (start 129.75 90.95) (end 131.4 89.3) (width 0.25) (layer "B.Cu") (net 26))
 (segment (start 151.8 89.3) (end 153.25 90.75) (width 0.25) (layer "B.Cu") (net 26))
 (segment (start 120.8 91.5) (end 120.8 93.225) (width 0.25) (layer "F.Cu") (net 2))
 (segment (start 120.8 93.225) (end 121.75 94.175) (width 0.25) (layer "F.Cu") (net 2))
 (segment (start 174.0625 99.75) (end 155.5 99.75) (width 0.25) (layer "B.Cu") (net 2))
 (segment (start 155.5 99.75) (end 155.25 100) (width 0.25) (layer "B.Cu") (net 2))
 (segment (start 155.25 100) (end 151.36525 100) (width 0.25) (layer "B.Cu") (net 2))
 (via (at 169.25 100.5) (size 0.8) (drill 0.4) (layers "F.Cu" "B.Cu") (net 19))
 (segment (start 174.0625 100.25) (end 169.5 100.25) (width 0.25) (layer "B.Cu") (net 19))
 (segment (start 169.5 100.25) (end 169.25 100.5) (width 0.25) (layer "B.Cu") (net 19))
 (segment (start 162.75 109.75) (end 162.75 108.15) (width 0.25) (layer "B.Cu") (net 16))
 (segment (start 150.9 107) (end 154.25 107) (width 0.25) (layer "B.Cu") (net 16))
 (segment (start 154.25 107) (end 157.375 110.125) (width 0.25) (layer "B.Cu") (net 16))
 (segment (start 162.375 110.125) (end 162.75 109.75) (width 0.25) (layer "B.Cu") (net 16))
 (segment (start 157.375 110.125) (end 162.375 110.125) (width 0.25) (layer "B.Cu") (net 16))
 (segment (start 150.9 107.5) (end 154 107.5) (width 0.25) (layer "B.Cu") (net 20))
 (segment (start 157.25 110.75) (end 169.5 110.75) (width 0.25) (layer "B.Cu") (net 20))
 (segment (start 169.5 110.75) (end 170.25 110) (width 0.25) (layer "B.Cu") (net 20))
 (segment (start 154 107.5) (end 157.25 110.75) (width 0.25) (layer "B.Cu") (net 20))
 (segment (start 170.25 110) (end 170.25 108.15) (width 0.25) (layer "B.Cu") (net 20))
 (segment (start 120 100.957538) (end 120 101.25) (width 0.25) (layer "F.Cu") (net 6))
 (segment (start 121.25 99) (end 121.25 99.707538) (width 0.25) (layer "F.Cu") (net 6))
 (segment (start 121.25 99.707538) (end 120 100.957538) (width 0.25) (layer "F.Cu") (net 6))
 (via (at 120 101.25) (size 0.8) (drill 0.4) (layers "F.Cu" "B.Cu") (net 6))
 (segment (start 120 102.75) (end 120 101.25) (width 0.25) (layer "B.Cu") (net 6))
 (segment (start 118.4625 108.75) (end 118.4625 104.2875) (width 0.25) (layer "B.Cu") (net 6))
 (segment (start 118.4625 104.2875) (end 120 102.75) (width 0.25) (layer "B.Cu") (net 6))
 (segment (start 120.0375 108.75) (end 121.925 108.75) (width 0.25) (layer "B.Cu") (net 22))
 (segment (start 118.5 93.25) (end 118.5 92.75) (width 0.25) (layer "F.Cu") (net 5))
 (segment (start 119.25 96.75) (end 119.25 94.5) (width 0.25) (layer "F.Cu") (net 5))
 (segment (start 119.25 97.874998) (end 119.25 96.75) (width 0.25) (layer "F.Cu") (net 5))
 (segment (start 120.750001 99) (end 120.375002 99) (width 0.25) (layer "F.Cu") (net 5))
 (segment (start 119.25 94) (end 118.75 93.5) (width 0.25) (layer "F.Cu") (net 5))
 (segment (start 119.25 94.5) (end 119.25 94) (width 0.25) (layer "F.Cu") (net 5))
 (segment (start 120.375002 99) (end 119.25 97.874998) (width 0.25) (layer "F.Cu") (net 5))
 (segment (start 118.75 93.5) (end 118.5 93.25) (width 0.25) (layer "F.Cu") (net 5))
 (via (at 118.5 92.75) (size 0.8) (drill 0.4) (layers "F.Cu" "B.Cu") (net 5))
 (segment (start 118.5 91.2875) (end 118.4625 91.25) (width 0.25) (layer "B.Cu") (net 5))
 (segment (start 118.5 92.75) (end 118.5 91.2875) (width 0.25) (layer "B.Cu") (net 5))
 (segment (start 120.0375 91.25) (end 121.925 91.25) (width 0.25) (layer "B.Cu") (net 41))
 (segment (start 137 97.25) (end 174.0625 97.25) (width 0.25) (layer "B.Cu") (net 24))
 (segment (start 134.25 91.85) (end 134.25 94.5) (width 0.25) (layer "B.Cu") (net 24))
 (segment (start 134.25 94.5) (end 137 97.25) (width 0.25) (layer "B.Cu") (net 24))
 (segment (start 132.75 94) (end 136.5 97.75) (width 0.25) (layer "B.Cu") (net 25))
 (segment (start 132.75 91.85) (end 132.75 94) (width 0.25) (layer "B.Cu") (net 25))
 (segment (start 136.5 97.75) (end 174.0625 97.75) (width 0.25) (layer "B.Cu") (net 25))
 (segment (start 168.5 102.25) (end 174.0625 102.25) (width 0.25) (layer "B.Cu") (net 17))
 (segment (start 165.75 105) (end 168.5 102.25) (width 0.25) (layer "B.Cu") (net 17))
 (segment (start 165.75 108.15) (end 165.75 105) (width 0.25) (layer "B.Cu") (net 17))
 (segment (start 169 102.75) (end 174.0625 102.75) (width 0.25) (layer "B.Cu") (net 18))
 (segment (start 167.25 108.15) (end 167.25 104.5) (width 0.25) (layer "B.Cu") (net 18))
 (segment (start 167.25 104.5) (end 169 102.75) (width 0.25) (layer "B.Cu") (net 18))
 (segment (start 121.750002 99) (end 121.750002 100.424998) (width 0.25) (layer "F.Cu") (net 7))
 (segment (start 121.750002 100.424998) (end 121.75 100.425) (width 0.25) (layer "F.Cu") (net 7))
 (segment (start 121.75 95.825) (end 121.75 97.099996) (width 0.25) (layer "F.Cu") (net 1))
 (segment (start 121.75 97.099996) (end 121.750002 97.099998) (width 0.25) (layer "F.Cu") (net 1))
 (segment (start 120.25 90.25) (end 119.85 90.65) (width 0.25) (layer "F.Cu") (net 8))
 (segment (start 122.25 99) (end 124.75 99) (width 0.25) (layer "F.Cu") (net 8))
 (segment (start 121.75 90.75) (end 121.25 90.25) (width 0.25) (layer "F.Cu") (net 8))
 (segment (start 124.75 99) (end 124.75 92) (width 0.25) (layer "F.Cu") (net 8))
 (segment (start 124.25 91.5) (end 124.75 92) (width 0.25) (layer "F.Cu") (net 8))
 (segment (start 121.75 91.5) (end 121.75 90.75) (width 0.25) (layer "F.Cu") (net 8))
 (segment (start 119.85 90.65) (end 119.85 91.5) (width 0.25) (layer "F.Cu") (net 8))
 (segment (start 124.75 108.25) (end 124.75 99) (width 0.25) (layer "F.Cu") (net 8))
 (segment (start 121.75 91.5) (end 124.25 91.5) (width 0.25) (layer "F.Cu") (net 8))
 (segment (start 121.25 90.25) (end 120.25 90.25) (width 0.25) (layer "F.Cu") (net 8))
 (via (at 124.75 92) (size 0.8) (drill 0.4) (layers "F.Cu" "B.Cu") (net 8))
 (via (at 124.75 108.25) (size 0.8) (drill 0.4) (layers "F.Cu" "B.Cu") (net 8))
 (segment (start 124.5 91.25) (end 123.575 91.25) (width 0.25) (layer "B.Cu") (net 8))
 (segment (start 123.575 108.75) (end 124.25 108.75) (width 0.25) (layer "B.Cu") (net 8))
 (segment (start 124.75 91.5) (end 124.5 91.25) (width 0.25) (layer "B.Cu") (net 8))
 (segment (start 124.75 92) (end 124.75 91.5) (width 0.25) (layer "B.Cu") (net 8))
 (segment (start 124.25 108.75) (end 124.75 108.25) (width 0.25) (layer "B.Cu") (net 8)))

